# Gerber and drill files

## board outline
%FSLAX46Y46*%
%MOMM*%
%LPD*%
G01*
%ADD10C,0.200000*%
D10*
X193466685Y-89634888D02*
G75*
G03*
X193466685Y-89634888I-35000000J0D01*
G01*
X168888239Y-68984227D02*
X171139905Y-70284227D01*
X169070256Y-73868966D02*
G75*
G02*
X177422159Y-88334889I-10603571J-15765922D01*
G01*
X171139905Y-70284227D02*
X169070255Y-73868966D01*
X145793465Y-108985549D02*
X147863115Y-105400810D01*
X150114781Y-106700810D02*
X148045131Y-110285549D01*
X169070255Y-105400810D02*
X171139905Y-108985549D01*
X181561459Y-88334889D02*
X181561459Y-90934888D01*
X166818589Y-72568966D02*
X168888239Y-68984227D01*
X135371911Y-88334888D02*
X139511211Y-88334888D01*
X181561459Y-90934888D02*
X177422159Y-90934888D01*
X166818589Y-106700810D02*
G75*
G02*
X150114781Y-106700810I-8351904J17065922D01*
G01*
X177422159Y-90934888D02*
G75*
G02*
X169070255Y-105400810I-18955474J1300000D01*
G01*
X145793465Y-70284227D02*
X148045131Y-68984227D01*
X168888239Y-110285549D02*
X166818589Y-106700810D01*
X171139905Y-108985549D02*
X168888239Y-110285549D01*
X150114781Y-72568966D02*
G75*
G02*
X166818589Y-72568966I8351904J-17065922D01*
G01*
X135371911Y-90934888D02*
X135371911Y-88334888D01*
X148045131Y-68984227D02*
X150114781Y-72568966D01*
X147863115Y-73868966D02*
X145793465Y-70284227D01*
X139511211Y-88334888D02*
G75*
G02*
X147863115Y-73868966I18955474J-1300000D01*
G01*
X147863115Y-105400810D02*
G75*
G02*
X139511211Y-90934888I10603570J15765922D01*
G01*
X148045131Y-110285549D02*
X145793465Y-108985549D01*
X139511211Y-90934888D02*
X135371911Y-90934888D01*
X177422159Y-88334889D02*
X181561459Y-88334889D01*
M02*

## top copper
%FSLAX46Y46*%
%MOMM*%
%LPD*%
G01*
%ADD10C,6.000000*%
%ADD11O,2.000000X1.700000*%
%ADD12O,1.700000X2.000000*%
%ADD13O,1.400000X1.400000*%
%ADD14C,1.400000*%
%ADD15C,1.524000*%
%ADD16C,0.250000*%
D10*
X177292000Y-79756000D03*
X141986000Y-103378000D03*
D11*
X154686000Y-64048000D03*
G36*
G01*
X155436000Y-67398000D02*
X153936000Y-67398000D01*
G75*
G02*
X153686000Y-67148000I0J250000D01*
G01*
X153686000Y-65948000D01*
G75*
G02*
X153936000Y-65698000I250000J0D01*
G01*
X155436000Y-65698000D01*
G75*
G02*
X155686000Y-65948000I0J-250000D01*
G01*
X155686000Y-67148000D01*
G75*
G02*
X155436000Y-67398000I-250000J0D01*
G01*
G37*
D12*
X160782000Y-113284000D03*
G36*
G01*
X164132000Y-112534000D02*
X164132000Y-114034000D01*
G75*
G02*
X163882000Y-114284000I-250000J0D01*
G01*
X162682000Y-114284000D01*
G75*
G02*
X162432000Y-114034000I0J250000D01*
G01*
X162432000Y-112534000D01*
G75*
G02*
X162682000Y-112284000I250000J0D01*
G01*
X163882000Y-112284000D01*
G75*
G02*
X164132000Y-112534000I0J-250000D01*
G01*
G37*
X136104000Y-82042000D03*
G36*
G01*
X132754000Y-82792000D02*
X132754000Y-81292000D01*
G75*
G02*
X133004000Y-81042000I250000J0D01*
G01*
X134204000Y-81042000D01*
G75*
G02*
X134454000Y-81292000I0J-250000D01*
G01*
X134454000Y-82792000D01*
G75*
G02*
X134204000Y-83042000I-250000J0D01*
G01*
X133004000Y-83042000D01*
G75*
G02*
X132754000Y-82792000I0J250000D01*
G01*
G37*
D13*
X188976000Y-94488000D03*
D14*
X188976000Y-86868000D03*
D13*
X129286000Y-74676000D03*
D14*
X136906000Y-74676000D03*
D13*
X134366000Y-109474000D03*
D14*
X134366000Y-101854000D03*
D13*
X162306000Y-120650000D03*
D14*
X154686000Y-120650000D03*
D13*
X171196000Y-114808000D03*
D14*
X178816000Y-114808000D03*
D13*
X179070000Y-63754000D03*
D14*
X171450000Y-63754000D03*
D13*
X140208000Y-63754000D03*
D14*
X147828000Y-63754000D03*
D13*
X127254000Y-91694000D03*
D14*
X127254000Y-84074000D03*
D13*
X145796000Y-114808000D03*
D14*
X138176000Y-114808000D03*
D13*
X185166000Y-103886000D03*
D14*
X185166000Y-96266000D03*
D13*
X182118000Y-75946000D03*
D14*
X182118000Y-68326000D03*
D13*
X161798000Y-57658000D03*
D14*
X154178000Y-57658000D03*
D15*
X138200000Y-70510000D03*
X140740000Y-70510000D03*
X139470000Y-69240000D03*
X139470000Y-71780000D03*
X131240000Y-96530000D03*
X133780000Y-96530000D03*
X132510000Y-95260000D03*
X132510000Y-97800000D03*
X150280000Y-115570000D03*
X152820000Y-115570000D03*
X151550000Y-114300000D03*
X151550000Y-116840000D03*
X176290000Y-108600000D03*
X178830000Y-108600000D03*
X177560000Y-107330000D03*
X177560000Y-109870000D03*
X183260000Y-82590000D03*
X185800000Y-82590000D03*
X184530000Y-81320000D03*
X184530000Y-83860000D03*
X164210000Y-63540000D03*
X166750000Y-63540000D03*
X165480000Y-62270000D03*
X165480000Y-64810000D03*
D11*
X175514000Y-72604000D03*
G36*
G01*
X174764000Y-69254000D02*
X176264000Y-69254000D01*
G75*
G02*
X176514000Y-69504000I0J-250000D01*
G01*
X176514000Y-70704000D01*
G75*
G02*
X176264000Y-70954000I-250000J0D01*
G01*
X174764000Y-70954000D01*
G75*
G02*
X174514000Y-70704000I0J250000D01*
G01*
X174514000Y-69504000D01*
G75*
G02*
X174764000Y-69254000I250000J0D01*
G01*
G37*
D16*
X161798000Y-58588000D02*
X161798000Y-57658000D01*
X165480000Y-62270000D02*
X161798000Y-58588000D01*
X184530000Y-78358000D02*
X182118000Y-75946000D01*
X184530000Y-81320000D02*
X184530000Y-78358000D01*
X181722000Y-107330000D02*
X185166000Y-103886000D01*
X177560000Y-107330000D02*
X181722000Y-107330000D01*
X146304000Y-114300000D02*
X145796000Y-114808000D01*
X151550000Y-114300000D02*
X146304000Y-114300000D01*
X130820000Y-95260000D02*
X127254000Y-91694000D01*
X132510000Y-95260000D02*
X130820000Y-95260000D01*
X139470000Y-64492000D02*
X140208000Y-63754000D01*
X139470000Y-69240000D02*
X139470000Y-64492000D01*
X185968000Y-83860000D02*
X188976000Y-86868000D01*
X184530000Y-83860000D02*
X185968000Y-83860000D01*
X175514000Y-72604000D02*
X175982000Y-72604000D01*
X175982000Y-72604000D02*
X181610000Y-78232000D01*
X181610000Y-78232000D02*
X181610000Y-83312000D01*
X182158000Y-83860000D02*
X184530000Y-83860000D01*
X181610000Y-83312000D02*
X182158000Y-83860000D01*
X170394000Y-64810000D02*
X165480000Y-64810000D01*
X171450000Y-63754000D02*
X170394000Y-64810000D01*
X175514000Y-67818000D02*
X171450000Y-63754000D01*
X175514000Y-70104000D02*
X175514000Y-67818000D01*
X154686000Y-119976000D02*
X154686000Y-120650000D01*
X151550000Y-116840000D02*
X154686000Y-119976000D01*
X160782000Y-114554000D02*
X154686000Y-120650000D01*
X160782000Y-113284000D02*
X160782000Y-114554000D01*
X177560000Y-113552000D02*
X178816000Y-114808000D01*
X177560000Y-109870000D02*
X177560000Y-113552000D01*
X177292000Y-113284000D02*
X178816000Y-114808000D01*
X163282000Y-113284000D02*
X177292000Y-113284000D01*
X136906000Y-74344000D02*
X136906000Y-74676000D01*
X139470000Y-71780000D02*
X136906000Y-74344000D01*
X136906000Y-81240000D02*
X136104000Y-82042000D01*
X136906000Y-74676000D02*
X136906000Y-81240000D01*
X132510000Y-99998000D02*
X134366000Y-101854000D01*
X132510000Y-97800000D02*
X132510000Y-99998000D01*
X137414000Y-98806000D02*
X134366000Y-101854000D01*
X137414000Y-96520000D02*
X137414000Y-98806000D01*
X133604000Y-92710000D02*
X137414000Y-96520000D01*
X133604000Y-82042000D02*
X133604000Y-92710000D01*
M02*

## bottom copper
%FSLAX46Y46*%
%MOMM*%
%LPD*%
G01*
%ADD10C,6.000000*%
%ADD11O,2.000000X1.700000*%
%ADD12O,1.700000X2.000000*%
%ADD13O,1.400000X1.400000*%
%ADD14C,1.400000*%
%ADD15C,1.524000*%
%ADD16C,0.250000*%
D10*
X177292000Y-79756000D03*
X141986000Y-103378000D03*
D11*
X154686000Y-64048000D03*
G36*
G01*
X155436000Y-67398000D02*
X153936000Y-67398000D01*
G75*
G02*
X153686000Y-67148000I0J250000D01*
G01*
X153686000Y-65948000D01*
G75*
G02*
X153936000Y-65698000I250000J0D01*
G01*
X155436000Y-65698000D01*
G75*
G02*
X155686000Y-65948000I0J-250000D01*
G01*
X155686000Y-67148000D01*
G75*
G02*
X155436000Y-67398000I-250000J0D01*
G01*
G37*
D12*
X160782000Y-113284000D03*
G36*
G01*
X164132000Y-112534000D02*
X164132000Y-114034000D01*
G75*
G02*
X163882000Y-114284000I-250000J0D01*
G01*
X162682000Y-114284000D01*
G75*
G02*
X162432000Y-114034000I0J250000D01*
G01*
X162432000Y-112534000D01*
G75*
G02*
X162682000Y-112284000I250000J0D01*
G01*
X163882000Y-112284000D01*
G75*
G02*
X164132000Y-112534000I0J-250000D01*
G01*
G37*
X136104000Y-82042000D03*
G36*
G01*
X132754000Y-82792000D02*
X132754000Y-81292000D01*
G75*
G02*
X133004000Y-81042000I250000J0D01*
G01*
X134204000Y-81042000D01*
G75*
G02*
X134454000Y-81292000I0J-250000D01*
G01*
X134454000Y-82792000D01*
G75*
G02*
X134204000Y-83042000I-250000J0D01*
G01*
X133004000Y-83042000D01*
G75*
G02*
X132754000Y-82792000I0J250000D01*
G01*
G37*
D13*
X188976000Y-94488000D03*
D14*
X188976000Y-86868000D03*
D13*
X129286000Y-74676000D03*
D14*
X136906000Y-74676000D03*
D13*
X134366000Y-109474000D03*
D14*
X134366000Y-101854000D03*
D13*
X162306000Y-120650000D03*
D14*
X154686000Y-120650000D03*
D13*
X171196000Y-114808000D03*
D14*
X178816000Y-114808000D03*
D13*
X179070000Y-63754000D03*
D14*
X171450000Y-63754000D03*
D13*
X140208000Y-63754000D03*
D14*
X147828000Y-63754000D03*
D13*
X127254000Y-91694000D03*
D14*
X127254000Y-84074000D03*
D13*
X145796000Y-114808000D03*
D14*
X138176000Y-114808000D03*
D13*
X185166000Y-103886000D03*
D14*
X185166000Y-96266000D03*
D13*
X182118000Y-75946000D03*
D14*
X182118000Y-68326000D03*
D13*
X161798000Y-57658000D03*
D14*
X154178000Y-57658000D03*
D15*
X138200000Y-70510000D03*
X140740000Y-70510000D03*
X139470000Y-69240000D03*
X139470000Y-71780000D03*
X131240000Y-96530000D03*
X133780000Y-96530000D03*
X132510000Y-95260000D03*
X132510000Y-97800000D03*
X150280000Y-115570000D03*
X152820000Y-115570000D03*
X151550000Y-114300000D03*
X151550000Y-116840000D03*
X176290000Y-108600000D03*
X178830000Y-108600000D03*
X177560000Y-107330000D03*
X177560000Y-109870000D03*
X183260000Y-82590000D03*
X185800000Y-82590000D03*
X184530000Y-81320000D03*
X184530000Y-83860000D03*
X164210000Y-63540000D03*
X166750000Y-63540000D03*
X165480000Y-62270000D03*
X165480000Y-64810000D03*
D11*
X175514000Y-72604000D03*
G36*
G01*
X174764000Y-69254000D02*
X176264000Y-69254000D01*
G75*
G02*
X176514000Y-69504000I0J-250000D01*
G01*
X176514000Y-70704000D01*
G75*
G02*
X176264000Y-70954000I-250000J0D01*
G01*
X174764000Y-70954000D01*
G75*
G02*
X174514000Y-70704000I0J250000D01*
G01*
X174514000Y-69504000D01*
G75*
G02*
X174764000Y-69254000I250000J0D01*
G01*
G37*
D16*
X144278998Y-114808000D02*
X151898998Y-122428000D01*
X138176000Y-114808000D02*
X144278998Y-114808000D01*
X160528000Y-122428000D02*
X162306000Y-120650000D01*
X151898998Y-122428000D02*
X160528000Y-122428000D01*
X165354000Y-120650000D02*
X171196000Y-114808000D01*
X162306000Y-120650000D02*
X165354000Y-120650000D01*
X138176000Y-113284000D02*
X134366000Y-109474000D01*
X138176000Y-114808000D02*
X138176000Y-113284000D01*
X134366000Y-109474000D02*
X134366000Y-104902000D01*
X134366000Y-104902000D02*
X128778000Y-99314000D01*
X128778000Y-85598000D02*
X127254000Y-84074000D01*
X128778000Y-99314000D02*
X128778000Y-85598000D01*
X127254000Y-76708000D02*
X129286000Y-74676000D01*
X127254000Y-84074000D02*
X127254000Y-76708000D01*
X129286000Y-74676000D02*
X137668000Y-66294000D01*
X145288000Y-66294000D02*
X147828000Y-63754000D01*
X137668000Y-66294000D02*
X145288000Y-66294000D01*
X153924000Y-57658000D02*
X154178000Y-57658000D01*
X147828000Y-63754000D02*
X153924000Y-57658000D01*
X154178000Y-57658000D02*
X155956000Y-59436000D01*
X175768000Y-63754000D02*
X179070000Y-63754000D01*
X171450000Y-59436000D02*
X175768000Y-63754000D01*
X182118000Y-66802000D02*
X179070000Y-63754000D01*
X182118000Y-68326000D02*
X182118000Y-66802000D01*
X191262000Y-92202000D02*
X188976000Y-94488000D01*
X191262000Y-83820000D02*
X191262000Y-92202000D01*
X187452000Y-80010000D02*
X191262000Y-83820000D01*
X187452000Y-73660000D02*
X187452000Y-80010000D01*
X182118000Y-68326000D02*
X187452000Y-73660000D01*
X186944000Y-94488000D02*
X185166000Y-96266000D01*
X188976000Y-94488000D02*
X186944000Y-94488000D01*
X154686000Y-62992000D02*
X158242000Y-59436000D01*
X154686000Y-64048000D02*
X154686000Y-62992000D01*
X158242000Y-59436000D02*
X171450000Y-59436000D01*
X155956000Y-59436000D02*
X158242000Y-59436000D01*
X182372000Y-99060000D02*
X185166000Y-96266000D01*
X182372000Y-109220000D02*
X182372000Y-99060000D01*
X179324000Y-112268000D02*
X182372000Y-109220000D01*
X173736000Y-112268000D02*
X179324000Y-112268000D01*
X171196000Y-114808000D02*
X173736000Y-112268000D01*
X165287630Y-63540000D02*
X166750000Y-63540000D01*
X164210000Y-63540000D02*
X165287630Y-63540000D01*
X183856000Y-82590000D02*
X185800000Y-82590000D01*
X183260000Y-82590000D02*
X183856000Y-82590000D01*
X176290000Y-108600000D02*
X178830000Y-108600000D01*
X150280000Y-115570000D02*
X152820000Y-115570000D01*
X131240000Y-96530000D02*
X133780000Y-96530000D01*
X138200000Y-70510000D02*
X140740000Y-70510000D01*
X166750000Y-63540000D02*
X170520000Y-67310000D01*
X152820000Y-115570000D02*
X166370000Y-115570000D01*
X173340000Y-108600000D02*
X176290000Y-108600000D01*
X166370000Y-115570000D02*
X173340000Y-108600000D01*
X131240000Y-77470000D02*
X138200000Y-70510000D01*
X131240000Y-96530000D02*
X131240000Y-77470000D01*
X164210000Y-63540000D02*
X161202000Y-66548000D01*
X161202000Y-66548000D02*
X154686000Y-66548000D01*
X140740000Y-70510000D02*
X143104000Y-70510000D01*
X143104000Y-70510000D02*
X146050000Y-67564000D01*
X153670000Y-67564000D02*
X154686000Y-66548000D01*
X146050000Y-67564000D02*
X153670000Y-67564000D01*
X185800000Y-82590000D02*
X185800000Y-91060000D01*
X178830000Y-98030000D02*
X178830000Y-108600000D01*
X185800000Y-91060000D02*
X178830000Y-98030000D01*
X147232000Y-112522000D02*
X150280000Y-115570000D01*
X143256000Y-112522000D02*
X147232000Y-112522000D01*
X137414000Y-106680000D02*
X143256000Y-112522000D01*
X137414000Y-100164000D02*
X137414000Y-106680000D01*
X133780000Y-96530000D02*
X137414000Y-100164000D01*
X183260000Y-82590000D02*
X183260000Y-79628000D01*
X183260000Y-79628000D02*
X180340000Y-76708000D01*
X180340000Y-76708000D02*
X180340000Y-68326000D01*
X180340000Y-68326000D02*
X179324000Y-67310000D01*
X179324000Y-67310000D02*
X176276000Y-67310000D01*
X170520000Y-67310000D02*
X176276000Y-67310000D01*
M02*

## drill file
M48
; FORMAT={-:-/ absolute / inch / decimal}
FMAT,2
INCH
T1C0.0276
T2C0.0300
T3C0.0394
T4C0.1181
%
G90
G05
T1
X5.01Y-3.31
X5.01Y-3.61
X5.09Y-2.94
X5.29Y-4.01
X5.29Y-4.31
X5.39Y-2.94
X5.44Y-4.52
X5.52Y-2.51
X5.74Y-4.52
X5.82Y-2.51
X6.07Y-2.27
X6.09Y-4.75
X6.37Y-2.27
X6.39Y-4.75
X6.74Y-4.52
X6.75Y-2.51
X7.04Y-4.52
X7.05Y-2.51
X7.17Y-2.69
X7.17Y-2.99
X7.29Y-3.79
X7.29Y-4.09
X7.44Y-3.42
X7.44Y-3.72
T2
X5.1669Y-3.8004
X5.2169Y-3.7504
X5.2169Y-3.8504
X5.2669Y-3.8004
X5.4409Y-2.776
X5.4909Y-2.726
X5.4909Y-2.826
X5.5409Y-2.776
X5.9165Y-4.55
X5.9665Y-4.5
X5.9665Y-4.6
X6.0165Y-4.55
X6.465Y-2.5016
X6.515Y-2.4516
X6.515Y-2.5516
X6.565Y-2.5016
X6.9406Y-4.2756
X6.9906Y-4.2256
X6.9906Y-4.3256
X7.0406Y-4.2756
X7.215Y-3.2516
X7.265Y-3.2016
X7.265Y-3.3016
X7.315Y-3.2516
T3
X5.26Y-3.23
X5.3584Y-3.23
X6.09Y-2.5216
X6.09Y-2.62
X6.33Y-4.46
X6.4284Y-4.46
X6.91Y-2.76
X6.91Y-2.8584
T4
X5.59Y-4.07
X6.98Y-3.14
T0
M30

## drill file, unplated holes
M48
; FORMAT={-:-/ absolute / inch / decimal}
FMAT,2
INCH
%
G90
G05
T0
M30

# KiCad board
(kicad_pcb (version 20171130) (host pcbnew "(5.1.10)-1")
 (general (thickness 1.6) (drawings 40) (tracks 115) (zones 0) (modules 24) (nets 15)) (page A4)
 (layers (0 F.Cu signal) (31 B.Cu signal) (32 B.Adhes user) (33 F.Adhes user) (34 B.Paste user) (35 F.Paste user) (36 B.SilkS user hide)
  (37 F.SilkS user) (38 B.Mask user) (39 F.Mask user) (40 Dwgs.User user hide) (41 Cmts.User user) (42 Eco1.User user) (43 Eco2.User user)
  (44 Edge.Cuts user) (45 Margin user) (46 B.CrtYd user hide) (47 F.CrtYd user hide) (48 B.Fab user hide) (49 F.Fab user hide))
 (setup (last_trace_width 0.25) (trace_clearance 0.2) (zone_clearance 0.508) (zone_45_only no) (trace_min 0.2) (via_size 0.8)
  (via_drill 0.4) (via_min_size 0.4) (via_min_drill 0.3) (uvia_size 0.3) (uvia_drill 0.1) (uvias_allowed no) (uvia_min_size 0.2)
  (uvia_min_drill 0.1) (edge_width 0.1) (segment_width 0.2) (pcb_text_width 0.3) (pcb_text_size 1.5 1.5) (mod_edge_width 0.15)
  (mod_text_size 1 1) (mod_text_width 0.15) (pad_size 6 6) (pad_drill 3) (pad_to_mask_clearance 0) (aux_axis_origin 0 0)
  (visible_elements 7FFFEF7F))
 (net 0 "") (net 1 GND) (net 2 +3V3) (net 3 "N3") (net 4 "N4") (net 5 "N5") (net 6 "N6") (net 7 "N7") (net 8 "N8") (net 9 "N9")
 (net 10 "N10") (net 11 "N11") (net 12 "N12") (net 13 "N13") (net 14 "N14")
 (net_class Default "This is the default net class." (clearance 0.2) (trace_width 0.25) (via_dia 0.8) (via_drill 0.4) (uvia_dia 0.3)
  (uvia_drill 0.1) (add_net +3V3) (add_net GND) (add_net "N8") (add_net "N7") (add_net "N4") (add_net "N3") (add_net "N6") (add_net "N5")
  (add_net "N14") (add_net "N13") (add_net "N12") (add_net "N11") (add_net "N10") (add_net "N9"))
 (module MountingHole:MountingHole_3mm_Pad (layer F.Cu) (at 177.292 79.756)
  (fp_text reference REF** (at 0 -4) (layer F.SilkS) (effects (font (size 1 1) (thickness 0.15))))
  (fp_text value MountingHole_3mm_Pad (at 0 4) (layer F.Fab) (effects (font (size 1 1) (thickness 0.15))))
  (pad "" thru_hole circle (at 0 0) (size 6 6) (drill 3) (layers *.Cu *.Mask)))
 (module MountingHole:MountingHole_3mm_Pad (layer F.Cu) (at 141.986 103.378)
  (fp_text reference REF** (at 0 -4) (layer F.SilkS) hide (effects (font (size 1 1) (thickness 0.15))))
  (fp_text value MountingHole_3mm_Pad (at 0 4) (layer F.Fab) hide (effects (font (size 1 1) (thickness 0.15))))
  (pad "" thru_hole circle (at 0 0) (size 6 6) (drill 3) (layers *.Cu *.Mask)))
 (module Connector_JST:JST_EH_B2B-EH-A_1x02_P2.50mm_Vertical (layer F.Cu) (at 154.686 66.548 90)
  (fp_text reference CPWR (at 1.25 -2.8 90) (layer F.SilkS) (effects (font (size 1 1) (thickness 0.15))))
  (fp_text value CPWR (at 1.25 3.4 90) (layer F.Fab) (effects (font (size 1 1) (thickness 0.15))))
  (pad 2 thru_hole oval (at 2.5 0 90) (size 1.7 2) (drill 1) (layers *.Cu *.Mask) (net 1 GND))
  (pad 1 thru_hole roundrect (at 0 0 90) (size 1.7 2) (drill 1) (layers *.Cu *.Mask) (roundrect_rratio 0.1470588235294118) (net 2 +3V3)))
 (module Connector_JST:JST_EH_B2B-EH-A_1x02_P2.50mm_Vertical (layer F.Cu) (at 163.282 113.284 180)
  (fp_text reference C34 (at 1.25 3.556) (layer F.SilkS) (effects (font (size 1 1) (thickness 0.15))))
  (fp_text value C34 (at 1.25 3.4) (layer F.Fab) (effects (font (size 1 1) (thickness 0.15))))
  (pad 2 thru_hole oval (at 2.5 0 180) (size 1.7 2) (drill 1) (layers *.Cu *.Mask) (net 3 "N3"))
  (pad 1 thru_hole roundrect (at 0 0 180) (size 1.7 2) (drill 1) (layers *.Cu *.Mask) (roundrect_rratio 0.1470588235294118) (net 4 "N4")))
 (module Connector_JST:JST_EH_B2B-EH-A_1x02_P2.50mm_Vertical (layer F.Cu) (at 133.604 82.042)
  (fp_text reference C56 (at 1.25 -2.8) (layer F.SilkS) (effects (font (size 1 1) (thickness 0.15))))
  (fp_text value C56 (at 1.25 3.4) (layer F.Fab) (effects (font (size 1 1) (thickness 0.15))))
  (pad 2 thru_hole oval (at 2.5 0) (size 1.7 2) (drill 1) (layers *.Cu *.Mask) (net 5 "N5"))
  (pad 1 thru_hole roundrect (at 0 0) (size 1.7 2) (drill 1) (layers *.Cu *.Mask) (roundrect_rratio 0.1470588235294118) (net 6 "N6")))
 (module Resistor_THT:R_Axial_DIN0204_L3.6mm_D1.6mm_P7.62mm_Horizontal (layer F.Cu) (at 188.976 86.868 270)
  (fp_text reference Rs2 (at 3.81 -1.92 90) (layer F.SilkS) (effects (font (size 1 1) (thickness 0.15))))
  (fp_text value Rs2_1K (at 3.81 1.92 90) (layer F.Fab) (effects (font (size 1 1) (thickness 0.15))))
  (pad 2 thru_hole oval (at 7.62 0 270) (size 1.4 1.4) (drill 0.7) (layers *.Cu *.Mask) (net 1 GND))
  (pad 1 thru_hole circle (at 0 0 270) (size 1.4 1.4) (drill 0.7) (layers *.Cu *.Mask) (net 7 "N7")))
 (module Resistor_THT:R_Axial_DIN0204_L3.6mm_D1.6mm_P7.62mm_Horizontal (layer F.Cu) (at 136.906 74.676 180)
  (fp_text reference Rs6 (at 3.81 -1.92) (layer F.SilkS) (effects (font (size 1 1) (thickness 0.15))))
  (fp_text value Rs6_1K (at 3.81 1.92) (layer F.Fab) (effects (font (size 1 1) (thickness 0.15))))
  (pad 2 thru_hole oval (at 7.62 0 180) (size 1.4 1.4) (drill 0.7) (layers *.Cu *.Mask) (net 1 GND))
  (pad 1 thru_hole circle (at 0 0 180) (size 1.4 1.4) (drill 0.7) (layers *.Cu *.Mask) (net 5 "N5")))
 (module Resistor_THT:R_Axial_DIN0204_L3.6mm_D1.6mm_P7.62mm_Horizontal (layer F.Cu) (at 134.366 101.854 270)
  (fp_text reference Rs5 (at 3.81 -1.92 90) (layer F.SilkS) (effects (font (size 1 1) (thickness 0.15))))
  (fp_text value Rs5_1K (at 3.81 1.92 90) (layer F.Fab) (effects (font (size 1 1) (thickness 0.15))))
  (pad 2 thru_hole oval (at 7.62 0 270) (size 1.4 1.4) (drill 0.7) (layers *.Cu *.Mask) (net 1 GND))
  (pad 1 thru_hole circle (at 0 0 270) (size 1.4 1.4) (drill 0.7) (layers *.Cu *.Mask) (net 6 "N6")))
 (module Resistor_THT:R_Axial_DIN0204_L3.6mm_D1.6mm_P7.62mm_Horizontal (layer F.Cu) (at 154.686 120.65)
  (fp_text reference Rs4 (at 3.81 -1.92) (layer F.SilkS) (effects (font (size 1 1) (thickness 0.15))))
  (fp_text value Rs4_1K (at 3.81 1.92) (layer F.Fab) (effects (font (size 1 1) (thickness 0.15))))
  (pad 2 thru_hole oval (at 7.62 0) (size 1.4 1.4) (drill 0.7) (layers *.Cu *.Mask) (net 1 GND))
  (pad 1 thru_hole circle (at 0 0) (size 1.4 1.4) (drill 0.7) (layers *.Cu *.Mask) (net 3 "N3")))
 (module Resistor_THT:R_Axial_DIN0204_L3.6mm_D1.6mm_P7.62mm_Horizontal (layer F.Cu) (at 178.816 114.808 180)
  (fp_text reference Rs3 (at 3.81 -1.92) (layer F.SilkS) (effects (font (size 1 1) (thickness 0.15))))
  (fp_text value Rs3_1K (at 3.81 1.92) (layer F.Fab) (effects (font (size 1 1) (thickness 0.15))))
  (pad 2 thru_hole oval (at 7.62 0 180) (size 1.4 1.4) (drill 0.7) (layers *.Cu *.Mask) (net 1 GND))
  (pad 1 thru_hole circle (at 0 0 180) (size 1.4 1.4) (drill 0.7) (layers *.Cu *.Mask) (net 4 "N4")))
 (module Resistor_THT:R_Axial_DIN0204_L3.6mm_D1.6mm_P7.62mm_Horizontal (layer F.Cu) (at 171.45 63.754)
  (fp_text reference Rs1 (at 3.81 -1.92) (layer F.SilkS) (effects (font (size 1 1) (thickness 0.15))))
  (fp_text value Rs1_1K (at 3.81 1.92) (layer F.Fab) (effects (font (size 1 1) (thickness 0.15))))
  (pad 2 thru_hole oval (at 7.62 0) (size 1.4 1.4) (drill 0.7) (layers *.Cu *.Mask) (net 1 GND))
  (pad 1 thru_hole circle (at 0 0) (size 1.4 1.4) (drill 0.7) (layers *.Cu *.Mask) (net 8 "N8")))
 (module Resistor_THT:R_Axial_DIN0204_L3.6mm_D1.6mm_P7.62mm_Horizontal (layer F.Cu) (at 147.828 63.754 180)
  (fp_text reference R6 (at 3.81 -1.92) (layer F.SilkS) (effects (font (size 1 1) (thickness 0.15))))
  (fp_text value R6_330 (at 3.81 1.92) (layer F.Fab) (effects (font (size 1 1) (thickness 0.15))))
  (pad 2 thru_hole oval (at 7.62 0 180) (size 1.4 1.4) (drill 0.7) (layers *.Cu *.Mask) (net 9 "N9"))
  (pad 1 thru_hole circle (at 0 0 180) (size 1.4 1.4) (drill 0.7) (layers *.Cu *.Mask) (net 1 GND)))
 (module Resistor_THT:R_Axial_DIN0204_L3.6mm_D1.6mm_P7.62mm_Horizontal (layer F.Cu) (at 127.254 84.074 270)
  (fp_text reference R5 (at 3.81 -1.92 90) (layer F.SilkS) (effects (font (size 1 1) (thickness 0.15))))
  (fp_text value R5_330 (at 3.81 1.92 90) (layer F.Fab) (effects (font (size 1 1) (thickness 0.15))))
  (pad 2 thru_hole oval (at 7.62 0 270) (size 1.4 1.4) (drill 0.7) (layers *.Cu *.Mask) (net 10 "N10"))
  (pad 1 thru_hole circle (at 0 0 270) (size 1.4 1.4) (drill 0.7) (layers *.Cu *.Mask) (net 1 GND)))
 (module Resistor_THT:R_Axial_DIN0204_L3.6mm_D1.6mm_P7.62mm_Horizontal (layer F.Cu) (at 138.176 114.808)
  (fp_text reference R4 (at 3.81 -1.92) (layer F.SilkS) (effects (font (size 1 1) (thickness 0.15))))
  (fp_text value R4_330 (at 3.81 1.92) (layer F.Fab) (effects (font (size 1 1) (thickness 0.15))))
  (pad 2 thru_hole oval (at 7.62 0) (size 1.4 1.4) (drill 0.7) (layers *.Cu *.Mask) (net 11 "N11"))
  (pad 1 thru_hole circle (at 0 0) (size 1.4 1.4) (drill 0.7) (layers *.Cu *.Mask) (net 1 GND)))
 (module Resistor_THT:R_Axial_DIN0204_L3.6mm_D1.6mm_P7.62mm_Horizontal (layer F.Cu) (at 185.166 96.266 270)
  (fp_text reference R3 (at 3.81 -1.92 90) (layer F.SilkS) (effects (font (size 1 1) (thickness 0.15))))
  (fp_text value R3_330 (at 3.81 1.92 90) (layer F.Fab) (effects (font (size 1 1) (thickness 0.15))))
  (pad 2 thru_hole oval (at 7.62 0 270) (size 1.4 1.4) (drill 0.7) (layers *.Cu *.Mask) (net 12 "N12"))
  (pad 1 thru_hole circle (at 0 0 270) (size 1.4 1.4) (drill 0.7) (layers *.Cu *.Mask) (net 1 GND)))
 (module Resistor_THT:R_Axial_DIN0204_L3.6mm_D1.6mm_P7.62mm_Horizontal (layer F.Cu) (at 182.118 68.326 270)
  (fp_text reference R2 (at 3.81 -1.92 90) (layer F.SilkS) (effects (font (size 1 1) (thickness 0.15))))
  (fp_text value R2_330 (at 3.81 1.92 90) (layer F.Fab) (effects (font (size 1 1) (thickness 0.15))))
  (pad 2 thru_hole oval (at 7.62 0 270) (size 1.4 1.4) (drill 0.7) (layers *.Cu *.Mask) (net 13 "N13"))
  (pad 1 thru_hole circle (at 0 0 270) (size 1.4 1.4) (drill 0.7) (layers *.Cu *.Mask) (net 1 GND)))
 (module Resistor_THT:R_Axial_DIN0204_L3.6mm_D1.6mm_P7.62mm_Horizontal (layer F.Cu) (at 154.178 57.658)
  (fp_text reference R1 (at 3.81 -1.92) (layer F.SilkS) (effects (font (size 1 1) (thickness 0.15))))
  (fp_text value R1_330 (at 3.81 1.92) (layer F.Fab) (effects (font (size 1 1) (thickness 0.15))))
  (pad 2 thru_hole oval (at 7.62 0) (size 1.4 1.4) (drill 0.7) (layers *.Cu *.Mask) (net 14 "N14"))
  (pad 1 thru_hole circle (at 0 0) (size 1.4 1.4) (drill 0.7) (layers *.Cu *.Mask) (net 1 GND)))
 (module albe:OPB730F (layer F.Cu) (at 139.47 70.51)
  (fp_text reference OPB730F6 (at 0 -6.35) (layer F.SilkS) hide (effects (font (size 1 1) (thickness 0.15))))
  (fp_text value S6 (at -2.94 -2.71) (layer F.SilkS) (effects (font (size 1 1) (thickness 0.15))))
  (pad 2 thru_hole circle (at -1.27 0) (size 1.524 1.524) (drill 0.762) (layers *.Cu *.Mask) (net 2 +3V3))
  (pad 4 thru_hole circle (at 1.27 0) (size 1.524 1.524) (drill 0.762) (layers *.Cu *.Mask) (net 2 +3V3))
  (pad 3 thru_hole circle (at 0 -1.27) (size 1.524 1.524) (drill 0.762) (layers *.Cu *.Mask) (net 9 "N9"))
  (pad 1 thru_hole circle (at 0 1.27) (size 1.524 1.524) (drill 0.762) (layers *.Cu *.Mask) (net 5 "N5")))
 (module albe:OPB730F (layer F.Cu) (at 132.51 96.53)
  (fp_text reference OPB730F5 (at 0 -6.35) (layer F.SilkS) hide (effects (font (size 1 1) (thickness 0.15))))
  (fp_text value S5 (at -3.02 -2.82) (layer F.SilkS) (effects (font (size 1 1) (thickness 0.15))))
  (pad 2 thru_hole circle (at -1.27 0) (size 1.524 1.524) (drill 0.762) (layers *.Cu *.Mask) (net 2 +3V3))
  (pad 4 thru_hole circle (at 1.27 0) (size 1.524 1.524) (drill 0.762) (layers *.Cu *.Mask) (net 2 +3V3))
  (pad 3 thru_hole circle (at 0 -1.27) (size 1.524 1.524) (drill 0.762) (layers *.Cu *.Mask) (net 10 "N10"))
  (pad 1 thru_hole circle (at 0 1.27) (size 1.524 1.524) (drill 0.762) (layers *.Cu *.Mask) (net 6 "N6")))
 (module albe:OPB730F (layer F.Cu) (at 151.55 115.57)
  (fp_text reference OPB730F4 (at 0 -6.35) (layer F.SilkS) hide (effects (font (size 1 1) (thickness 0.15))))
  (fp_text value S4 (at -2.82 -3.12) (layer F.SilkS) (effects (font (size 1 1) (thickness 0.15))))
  (pad 2 thru_hole circle (at -1.27 0) (size 1.524 1.524) (drill 0.762) (layers *.Cu *.Mask) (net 2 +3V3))
  (pad 4 thru_hole circle (at 1.27 0) (size 1.524 1.524) (drill 0.762) (layers *.Cu *.Mask) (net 2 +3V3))
  (pad 3 thru_hole circle (at 0 -1.27) (size 1.524 1.524) (drill 0.762) (layers *.Cu *.Mask) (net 11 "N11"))
  (pad 1 thru_hole circle (at 0 1.27) (size 1.524 1.524) (drill 0.762) (layers *.Cu *.Mask) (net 3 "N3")))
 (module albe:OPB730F (layer F.Cu) (at 177.56 108.6)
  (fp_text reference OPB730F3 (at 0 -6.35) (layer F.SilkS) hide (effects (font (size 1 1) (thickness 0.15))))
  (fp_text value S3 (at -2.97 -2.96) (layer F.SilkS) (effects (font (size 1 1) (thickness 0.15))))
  (pad 2 thru_hole circle (at -1.27 0) (size 1.524 1.524) (drill 0.762) (layers *.Cu *.Mask) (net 2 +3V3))
  (pad 4 thru_hole circle (at 1.27 0) (size 1.524 1.524) (drill 0.762) (layers *.Cu *.Mask) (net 2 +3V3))
  (pad 3 thru_hole circle (at 0 -1.27) (size 1.524 1.524) (drill 0.762) (layers *.Cu *.Mask) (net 12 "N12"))
  (pad 1 thru_hole circle (at 0 1.27) (size 1.524 1.524) (drill 0.762) (layers *.Cu *.Mask) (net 4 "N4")))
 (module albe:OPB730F (layer F.Cu) (at 184.53 82.59)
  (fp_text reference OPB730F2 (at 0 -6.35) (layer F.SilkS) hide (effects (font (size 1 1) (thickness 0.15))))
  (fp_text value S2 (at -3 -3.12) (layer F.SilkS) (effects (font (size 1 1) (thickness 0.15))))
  (pad 2 thru_hole circle (at -1.27 0) (size 1.524 1.524) (drill 0.762) (layers *.Cu *.Mask) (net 2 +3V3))
  (pad 4 thru_hole circle (at 1.27 0) (size 1.524 1.524) (drill 0.762) (layers *.Cu *.Mask) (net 2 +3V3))
  (pad 3 thru_hole circle (at 0 -1.27) (size 1.524 1.524) (drill 0.762) (layers *.Cu *.Mask) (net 13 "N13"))
  (pad 1 thru_hole circle (at 0 1.27) (size 1.524 1.524) (drill 0.762) (layers *.Cu *.Mask) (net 7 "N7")))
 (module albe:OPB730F (layer F.Cu) (at 165.48 63.54)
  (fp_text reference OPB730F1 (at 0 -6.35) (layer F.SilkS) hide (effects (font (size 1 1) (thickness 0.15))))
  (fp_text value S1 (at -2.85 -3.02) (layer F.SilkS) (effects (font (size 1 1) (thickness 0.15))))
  (pad 2 thru_hole circle (at -1.27 0) (size 1.524 1.524) (drill 0.762) (layers *.Cu *.Mask) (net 2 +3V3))
  (pad 4 thru_hole circle (at 1.27 0) (size 1.524 1.524) (drill 0.762) (layers *.Cu *.Mask) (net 2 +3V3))
  (pad 3 thru_hole circle (at 0 -1.27) (size 1.524 1.524) (drill 0.762) (layers *.Cu *.Mask) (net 14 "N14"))
  (pad 1 thru_hole circle (at 0 1.27) (size 1.524 1.524) (drill 0.762) (layers *.Cu *.Mask) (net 8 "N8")))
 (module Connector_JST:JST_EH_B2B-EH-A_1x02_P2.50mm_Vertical (layer F.Cu) (at 175.514 70.104 270)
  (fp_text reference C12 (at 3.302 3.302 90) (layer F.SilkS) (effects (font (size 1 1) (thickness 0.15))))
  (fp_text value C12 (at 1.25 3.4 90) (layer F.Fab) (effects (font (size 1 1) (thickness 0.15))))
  (pad 2 thru_hole oval (at 2.5 0 270) (size 1.7 2) (drill 1) (layers *.Cu *.Mask) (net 7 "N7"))
  (pad 1 thru_hole roundrect (at 0 0 270) (size 1.7 2) (drill 1) (layers *.Cu *.Mask) (roundrect_rratio 0.1470588235294118) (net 8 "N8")))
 (gr_circle (center 158.466685 89.634888) (end 193.466685 89.634888) (layer Edge.Cuts) (width 0.2))
 (gr_line (start 168.888239 68.984227) (end 171.139905 70.284227) (layer Edge.Cuts) (width 0.2))
 (gr_arc (start 158.466685 89.634888) (end 177.422159 88.334889) (angle -52.15339453) (layer Edge.Cuts) (width 0.2))
 (gr_line (start 171.139905 70.284227) (end 169.070255 73.868966) (layer Edge.Cuts) (width 0.2))
 (gr_line (start 145.793465 108.985549) (end 147.863115 105.40081) (layer Edge.Cuts) (width 0.2))
 (gr_line (start 150.114781 106.70081) (end 148.045131 110.285549) (layer Edge.Cuts) (width 0.2))
 (gr_line (start 169.070255 105.40081) (end 171.139905 108.985549) (layer Edge.Cuts) (width 0.2))
 (gr_line (start 181.561459 88.334889) (end 181.561459 90.934888) (layer Edge.Cuts) (width 0.2))
 (gr_line (start 166.818589 72.568966) (end 168.888239 68.984227) (layer Edge.Cuts) (width 0.2))
 (gr_line (start 135.371911 88.334888) (end 139.511211 88.334888) (layer Edge.Cuts) (width 0.2))
 (gr_line (start 181.561459 90.934888) (end 177.422159 90.934888) (layer Edge.Cuts) (width 0.2))
 (gr_arc (start 158.466685 89.634888) (end 150.114781 106.70081) (angle -52.15339453) (layer Edge.Cuts) (width 0.2))
 (gr_arc (start 158.466685 89.634888) (end 169.070255 105.40081) (angle -52.15339453) (layer Edge.Cuts) (width 0.2))
 (gr_line (start 145.793465 70.284227) (end 148.045131 68.984227) (layer Edge.Cuts) (width 0.2))
 (gr_line (start 168.888239 110.285549) (end 166.818589 106.70081) (layer Edge.Cuts) (width 0.2))
 (gr_line (start 171.139905 108.985549) (end 168.888239 110.285549) (layer Edge.Cuts) (width 0.2))
 (gr_arc (start 158.466685 89.634888) (end 166.818589 72.568966) (angle -52.15339453) (layer Edge.Cuts) (width 0.2))
 (gr_line (start 135.371911 90.934888) (end 135.371911 88.334888) (layer Edge.Cuts) (width 0.2))
 (gr_line (start 148.045131 68.984227) (end 150.114781 72.568966) (layer Edge.Cuts) (width 0.2))
 (gr_line (start 147.863115 73.868966) (end 145.793465 70.284227) (layer Edge.Cuts) (width 0.2))
 (gr_arc (start 158.466685 89.634888) (end 147.863115 73.868966) (angle -52.15339453) (layer Edge.Cuts) (width 0.2))
 (gr_arc (start 158.466685 89.634888) (end 139.511211 90.934888) (angle -52.15339453) (layer Edge.Cuts) (width 0.2))
 (gr_line (start 148.045131 110.285549) (end 145.793465 108.985549) (layer Edge.Cuts) (width 0.2))
 (gr_line (start 139.511211 90.934888) (end 135.371911 90.934888) (layer Edge.Cuts) (width 0.2))
 (gr_line (start 177.422159 88.334889) (end 181.561459 88.334889) (layer Edge.Cuts) (width 0.2))
 (segment (start 144.278998 114.808) (end 151.898998 122.428) (width 0.25) (layer B.Cu) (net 1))
 (segment (start 138.176 114.808) (end 144.278998 114.808) (width 0.25) (layer B.Cu) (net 1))
 (segment (start 160.528 122.428) (end 162.306 120.65) (width 0.25) (layer B.Cu) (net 1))
 (segment (start 151.898998 122.428) (end 160.528 122.428) (width 0.25) (layer B.Cu) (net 1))
 (segment (start 165.354 120.65) (end 171.196 114.808) (width 0.25) (layer B.Cu) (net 1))
 (segment (start 162.306 120.65) (end 165.354 120.65) (width 0.25) (layer B.Cu) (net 1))
 (segment (start 138.176 113.284) (end 134.366 109.474) (width 0.25) (layer B.Cu) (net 1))
 (segment (start 138.176 114.808) (end 138.176 113.284) (width 0.25) (layer B.Cu) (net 1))
 (segment (start 134.366 109.474) (end 134.366 104.902) (width 0.25) (layer B.Cu) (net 1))
 (segment (start 134.366 104.902) (end 128.778 99.314) (width 0.25) (layer B.Cu) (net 1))
 (segment (start 128.778 85.598) (end 127.254 84.074) (width 0.25) (layer B.Cu) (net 1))
 (segment (start 128.778 99.314) (end 128.778 85.598) (width 0.25) (layer B.Cu) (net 1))
 (segment (start 127.254 76.708) (end 129.286 74.676) (width 0.25) (layer B.Cu) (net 1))
 (segment (start 127.254 84.074) (end 127.254 76.708) (width 0.25) (layer B.Cu) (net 1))
 (segment (start 129.286 74.676) (end 137.668 66.294) (width 0.25) (layer B.Cu) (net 1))
 (segment (start 145.288 66.294) (end 147.828 63.754) (width 0.25) (layer B.Cu) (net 1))
 (segment (start 137.668 66.294) (end 145.288 66.294) (width 0.25) (layer B.Cu) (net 1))
 (segment (start 153.924 57.658) (end 154.178 57.658) (width 0.25) (layer B.Cu) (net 1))
 (segment (start 147.828 63.754) (end 153.924 57.658) (width 0.25) (layer B.Cu) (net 1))
 (segment (start 154.178 57.658) (end 155.956 59.436) (width 0.25) (layer B.Cu) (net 1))
 (segment (start 175.768 63.754) (end 179.07 63.754) (width 0.25) (layer B.Cu) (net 1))
 (segment (start 171.45 59.436) (end 175.768 63.754) (width 0.25) (layer B.Cu) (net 1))
 (segment (start 182.118 66.802) (end 179.07 63.754) (width 0.25) (layer B.Cu) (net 1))
 (segment (start 182.118 68.326) (end 182.118 66.802) (width 0.25) (layer B.Cu) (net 1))
 (segment (start 191.262 92.202) (end 188.976 94.488) (width 0.25) (layer B.Cu) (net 1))
 (segment (start 191.262 83.82) (end 191.262 92.202) (width 0.25) (layer B.Cu) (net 1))
 (segment (start 187.452 80.01) (end 191.262 83.82) (width 0.25) (layer B.Cu) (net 1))
 (segment (start 187.452 73.66) (end 187.452 80.01) (width 0.25) (layer B.Cu) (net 1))
 (segment (start 182.118 68.326) (end 187.452 73.66) (width 0.25) (layer B.Cu) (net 1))
 (segment (start 186.944 94.488) (end 185.166 96.266) (width 0.25) (layer B.Cu) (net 1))
 (segment (start 188.976 94.488) (end 186.944 94.488) (width 0.25) (layer B.Cu) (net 1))
 (segment (start 154.686 62.992) (end 158.242 59.436) (width 0.25) (layer B.Cu) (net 1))
 (segment (start 154.686 64.048) (end 154.686 62.992) (width 0.25) (layer B.Cu) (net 1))
 (segment (start 158.242 59.436) (end 171.45 59.436) (width 0.25) (layer B.Cu) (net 1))
 (segment (start 155.956 59.436) (end 158.242 59.436) (width 0.25) (layer B.Cu) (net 1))
 (segment (start 182.372 99.06) (end 185.166 96.266) (width 0.25) (layer B.Cu) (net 1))
 (segment (start 182.372 109.22) (end 182.372 99.06) (width 0.25) (layer B.Cu) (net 1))
 (segment (start 179.324 112.268) (end 182.372 109.22) (width 0.25) (layer B.Cu) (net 1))
 (segment (start 173.736 112.268) (end 179.324 112.268) (width 0.25) (layer B.Cu) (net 1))
 (segment (start 171.196 114.808) (end 173.736 112.268) (width 0.25) (layer B.Cu) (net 1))
 (segment (start 165.28763 63.54) (end 166.75 63.54) (width 0.25) (layer B.Cu) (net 2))
 (segment (start 164.21 63.54) (end 165.28763 63.54) (width 0.25) (layer B.Cu) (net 2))
 (segment (start 183.856 82.59) (end 185.8 82.59) (width 0.25) (layer B.Cu) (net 2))
 (segment (start 183.26 82.59) (end 183.856 82.59) (width 0.25) (layer B.Cu) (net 2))
 (segment (start 176.29 108.6) (end 178.83 108.6) (width 0.25) (layer B.Cu) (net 2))
 (segment (start 150.28 115.57) (end 152.82 115.57) (width 0.25) (layer B.Cu) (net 2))
 (segment (start 131.24 96.53) (end 133.78 96.53) (width 0.25) (layer B.Cu) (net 2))
 (segment (start 138.2 70.51) (end 140.74 70.51) (width 0.25) (layer B.Cu) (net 2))
 (segment (start 166.75 63.54) (end 170.52 67.31) (width 0.25) (layer B.Cu) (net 2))
 (segment (start 152.82 115.57) (end 166.37 115.57) (width 0.25) (layer B.Cu) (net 2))
 (segment (start 173.34 108.6) (end 176.29 108.6) (width 0.25) (layer B.Cu) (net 2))
 (segment (start 166.37 115.57) (end 173.34 108.6) (width 0.25) (layer B.Cu) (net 2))
 (segment (start 131.24 77.47) (end 138.2 70.51) (width 0.25) (layer B.Cu) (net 2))
 (segment (start 131.24 96.53) (end 131.24 77.47) (width 0.25) (layer B.Cu) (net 2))
 (segment (start 164.21 63.54) (end 161.202 66.548) (width 0.25) (layer B.Cu) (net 2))
 (segment (start 161.202 66.548) (end 154.686 66.548) (width 0.25) (layer B.Cu) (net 2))
 (segment (start 140.74 70.51) (end 143.104 70.51) (width 0.25) (layer B.Cu) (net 2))
 (segment (start 143.104 70.51) (end 146.05 67.564) (width 0.25) (layer B.Cu) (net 2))
 (segment (start 153.67 67.564) (end 154.686 66.548) (width 0.25) (layer B.Cu) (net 2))
 (segment (start 146.05 67.564) (end 153.67 67.564) (width 0.25) (layer B.Cu) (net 2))
 (segment (start 185.8 82.59) (end 185.8 91.06) (width 0.25) (layer B.Cu) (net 2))
 (segment (start 178.83 98.03) (end 178.83 108.6) (width 0.25) (layer B.Cu) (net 2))
 (segment (start 185.8 91.06) (end 178.83 98.03) (width 0.25) (layer B.Cu) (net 2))
 (segment (start 147.232 112.522) (end 150.28 115.57) (width 0.25) (layer B.Cu) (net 2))
 (segment (start 143.256 112.522) (end 147.232 112.522) (width 0.25) (layer B.Cu) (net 2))
 (segment (start 137.414 106.68) (end 143.256 112.522) (width 0.25) (layer B.Cu) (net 2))
 (segment (start 137.414 100.164) (end 137.414 106.68) (width 0.25) (layer B.Cu) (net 2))
 (segment (start 133.78 96.53) (end 137.414 100.164) (width 0.25) (layer B.Cu) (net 2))
 (segment (start 183.26 82.59) (end 183.26 79.628) (width 0.25) (layer B.Cu) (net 2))
 (segment (start 183.26 79.628) (end 180.34 76.708) (width 0.25) (layer B.Cu) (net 2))
 (segment (start 180.34 76.708) (end 180.34 68.326) (width 0.25) (layer B.Cu) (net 2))
 (segment (start 180.34 68.326) (end 179.324 67.31) (width 0.25) (layer B.Cu) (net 2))
 (segment (start 179.324 67.31) (end 176.276 67.31) (width 0.25) (layer B.Cu) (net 2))
 (segment (start 170.52 67.31) (end 176.276 67.31) (width 0.25) (layer B.Cu) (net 2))
 (segment (start 161.798 58.588) (end 161.798 57.658) (width 0.25) (layer F.Cu) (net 14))
 (segment (start 165.48 62.27) (end 161.798 58.588) (width 0.25) (layer F.Cu) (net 14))
 (segment (start 184.53 78.358) (end 182.118 75.946) (width 0.25) (layer F.Cu) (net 13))
 (segment (start 184.53 81.32) (end 184.53 78.358) (width 0.25) (layer F.Cu) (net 13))
 (segment (start 181.722 107.33) (end 185.166 103.886) (width 0.25) (layer F.Cu) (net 12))
 (segment (start 177.56 107.33) (end 181.722 107.33) (width 0.25) (layer F.Cu) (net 12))
 (segment (start 146.304 114.3) (end 145.796 114.808) (width 0.25) (layer F.Cu) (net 11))
 (segment (start 151.55 114.3) (end 146.304 114.3) (width 0.25) (layer F.Cu) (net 11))
 (segment (start 130.82 95.26) (end 127.254 91.694) (width 0.25) (layer F.Cu) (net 10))
 (segment (start 132.51 95.26) (end 130.82 95.26) (width 0.25) (layer F.Cu) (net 10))
 (segment (start 139.47 64.492) (end 140.208 63.754) (width 0.25) (layer F.Cu) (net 9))
 (segment (start 139.47 69.24) (end 139.47 64.492) (width 0.25) (layer F.Cu) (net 9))
 (segment (start 185.968 83.86) (end 188.976 86.868) (width 0.25) (layer F.Cu) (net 7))
 (segment (start 184.53 83.86) (end 185.968 83.86) (width 0.25) (layer F.Cu) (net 7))
 (segment (start 175.514 72.604) (end 175.982 72.604) (width 0.25) (layer F.Cu) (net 7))
 (segment (start 175.982 72.604) (end 181.61 78.232) (width 0.25) (layer F.Cu) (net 7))
 (segment (start 181.61 78.232) (end 181.61 83.312) (width 0.25) (layer F.Cu) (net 7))
 (segment (start 182.158 83.86) (end 184.53 83.86) (width 0.25) (layer F.Cu) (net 7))
 (segment (start 181.61 83.312) (end 182.158 83.86) (width 0.25) (layer F.Cu) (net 7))
 (segment (start 170.394 64.81) (end 165.48 64.81) (width 0.25) (layer F.Cu) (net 8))
 (segment (start 171.45 63.754) (end 170.394 64.81) (width 0.25) (layer F.Cu) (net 8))
 (segment (start 175.514 67.818) (end 171.45 63.754) (width 0.25) (layer F.Cu) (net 8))
 (segment (start 175.514 70.104) (end 175.514 67.818) (width 0.25) (layer F.Cu) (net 8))
 (segment (start 154.686 119.976) (end 154.686 120.65) (width 0.25) (layer F.Cu) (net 3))
 (segment (start 151.55 116.84) (end 154.686 119.976) (width 0.25) (layer F.Cu) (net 3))
 (segment (start 160.782 114.554) (end 154.686 120.65) (width 0.25) (layer F.Cu) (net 3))
 (segment (start 160.782 113.284) (end 160.782 114.554) (width 0.25) (layer F.Cu) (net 3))
 (segment (start 177.56 113.552) (end 178.816 114.808) (width 0.25) (layer F.Cu) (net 4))
 (segment (start 177.56 109.87) (end 177.56 113.552) (width 0.25) (layer F.Cu) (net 4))
 (segment (start 177.292 113.284) (end 178.816 114.808) (width 0.25) (layer F.Cu) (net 4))
 (segment (start 163.282 113.284) (end 177.292 113.284) (width 0.25) (layer F.Cu) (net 4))
 (segment (start 136.906 74.344) (end 136.906 74.676) (width 0.25) (layer F.Cu) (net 5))
 (segment (start 139.47 71.78) (end 136.906 74.344) (width 0.25) (layer F.Cu) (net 5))
 (segment (start 136.906 81.24) (end 136.104 82.042) (width 0.25) (layer F.Cu) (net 5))
 (segment (start 136.906 74.676) (end 136.906 81.24) (width 0.25) (layer F.Cu) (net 5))
 (segment (start 132.51 99.998) (end 134.366 101.854) (width 0.25) (layer F.Cu) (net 6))
 (segment (start 132.51 97.8) (end 132.51 99.998) (width 0.25) (layer F.Cu) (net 6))
 (segment (start 137.414 98.806) (end 134.366 101.854) (width 0.25) (layer F.Cu) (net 6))
 (segment (start 137.414 96.52) (end 137.414 98.806) (width 0.25) (layer F.Cu) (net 6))
 (segment (start 133.604 92.71) (end 137.414 96.52) (width 0.25) (layer F.Cu) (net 6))
 (segment (start 133.604 82.042) (end 133.604 92.71) (width 0.25) (layer F.Cu) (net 6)))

